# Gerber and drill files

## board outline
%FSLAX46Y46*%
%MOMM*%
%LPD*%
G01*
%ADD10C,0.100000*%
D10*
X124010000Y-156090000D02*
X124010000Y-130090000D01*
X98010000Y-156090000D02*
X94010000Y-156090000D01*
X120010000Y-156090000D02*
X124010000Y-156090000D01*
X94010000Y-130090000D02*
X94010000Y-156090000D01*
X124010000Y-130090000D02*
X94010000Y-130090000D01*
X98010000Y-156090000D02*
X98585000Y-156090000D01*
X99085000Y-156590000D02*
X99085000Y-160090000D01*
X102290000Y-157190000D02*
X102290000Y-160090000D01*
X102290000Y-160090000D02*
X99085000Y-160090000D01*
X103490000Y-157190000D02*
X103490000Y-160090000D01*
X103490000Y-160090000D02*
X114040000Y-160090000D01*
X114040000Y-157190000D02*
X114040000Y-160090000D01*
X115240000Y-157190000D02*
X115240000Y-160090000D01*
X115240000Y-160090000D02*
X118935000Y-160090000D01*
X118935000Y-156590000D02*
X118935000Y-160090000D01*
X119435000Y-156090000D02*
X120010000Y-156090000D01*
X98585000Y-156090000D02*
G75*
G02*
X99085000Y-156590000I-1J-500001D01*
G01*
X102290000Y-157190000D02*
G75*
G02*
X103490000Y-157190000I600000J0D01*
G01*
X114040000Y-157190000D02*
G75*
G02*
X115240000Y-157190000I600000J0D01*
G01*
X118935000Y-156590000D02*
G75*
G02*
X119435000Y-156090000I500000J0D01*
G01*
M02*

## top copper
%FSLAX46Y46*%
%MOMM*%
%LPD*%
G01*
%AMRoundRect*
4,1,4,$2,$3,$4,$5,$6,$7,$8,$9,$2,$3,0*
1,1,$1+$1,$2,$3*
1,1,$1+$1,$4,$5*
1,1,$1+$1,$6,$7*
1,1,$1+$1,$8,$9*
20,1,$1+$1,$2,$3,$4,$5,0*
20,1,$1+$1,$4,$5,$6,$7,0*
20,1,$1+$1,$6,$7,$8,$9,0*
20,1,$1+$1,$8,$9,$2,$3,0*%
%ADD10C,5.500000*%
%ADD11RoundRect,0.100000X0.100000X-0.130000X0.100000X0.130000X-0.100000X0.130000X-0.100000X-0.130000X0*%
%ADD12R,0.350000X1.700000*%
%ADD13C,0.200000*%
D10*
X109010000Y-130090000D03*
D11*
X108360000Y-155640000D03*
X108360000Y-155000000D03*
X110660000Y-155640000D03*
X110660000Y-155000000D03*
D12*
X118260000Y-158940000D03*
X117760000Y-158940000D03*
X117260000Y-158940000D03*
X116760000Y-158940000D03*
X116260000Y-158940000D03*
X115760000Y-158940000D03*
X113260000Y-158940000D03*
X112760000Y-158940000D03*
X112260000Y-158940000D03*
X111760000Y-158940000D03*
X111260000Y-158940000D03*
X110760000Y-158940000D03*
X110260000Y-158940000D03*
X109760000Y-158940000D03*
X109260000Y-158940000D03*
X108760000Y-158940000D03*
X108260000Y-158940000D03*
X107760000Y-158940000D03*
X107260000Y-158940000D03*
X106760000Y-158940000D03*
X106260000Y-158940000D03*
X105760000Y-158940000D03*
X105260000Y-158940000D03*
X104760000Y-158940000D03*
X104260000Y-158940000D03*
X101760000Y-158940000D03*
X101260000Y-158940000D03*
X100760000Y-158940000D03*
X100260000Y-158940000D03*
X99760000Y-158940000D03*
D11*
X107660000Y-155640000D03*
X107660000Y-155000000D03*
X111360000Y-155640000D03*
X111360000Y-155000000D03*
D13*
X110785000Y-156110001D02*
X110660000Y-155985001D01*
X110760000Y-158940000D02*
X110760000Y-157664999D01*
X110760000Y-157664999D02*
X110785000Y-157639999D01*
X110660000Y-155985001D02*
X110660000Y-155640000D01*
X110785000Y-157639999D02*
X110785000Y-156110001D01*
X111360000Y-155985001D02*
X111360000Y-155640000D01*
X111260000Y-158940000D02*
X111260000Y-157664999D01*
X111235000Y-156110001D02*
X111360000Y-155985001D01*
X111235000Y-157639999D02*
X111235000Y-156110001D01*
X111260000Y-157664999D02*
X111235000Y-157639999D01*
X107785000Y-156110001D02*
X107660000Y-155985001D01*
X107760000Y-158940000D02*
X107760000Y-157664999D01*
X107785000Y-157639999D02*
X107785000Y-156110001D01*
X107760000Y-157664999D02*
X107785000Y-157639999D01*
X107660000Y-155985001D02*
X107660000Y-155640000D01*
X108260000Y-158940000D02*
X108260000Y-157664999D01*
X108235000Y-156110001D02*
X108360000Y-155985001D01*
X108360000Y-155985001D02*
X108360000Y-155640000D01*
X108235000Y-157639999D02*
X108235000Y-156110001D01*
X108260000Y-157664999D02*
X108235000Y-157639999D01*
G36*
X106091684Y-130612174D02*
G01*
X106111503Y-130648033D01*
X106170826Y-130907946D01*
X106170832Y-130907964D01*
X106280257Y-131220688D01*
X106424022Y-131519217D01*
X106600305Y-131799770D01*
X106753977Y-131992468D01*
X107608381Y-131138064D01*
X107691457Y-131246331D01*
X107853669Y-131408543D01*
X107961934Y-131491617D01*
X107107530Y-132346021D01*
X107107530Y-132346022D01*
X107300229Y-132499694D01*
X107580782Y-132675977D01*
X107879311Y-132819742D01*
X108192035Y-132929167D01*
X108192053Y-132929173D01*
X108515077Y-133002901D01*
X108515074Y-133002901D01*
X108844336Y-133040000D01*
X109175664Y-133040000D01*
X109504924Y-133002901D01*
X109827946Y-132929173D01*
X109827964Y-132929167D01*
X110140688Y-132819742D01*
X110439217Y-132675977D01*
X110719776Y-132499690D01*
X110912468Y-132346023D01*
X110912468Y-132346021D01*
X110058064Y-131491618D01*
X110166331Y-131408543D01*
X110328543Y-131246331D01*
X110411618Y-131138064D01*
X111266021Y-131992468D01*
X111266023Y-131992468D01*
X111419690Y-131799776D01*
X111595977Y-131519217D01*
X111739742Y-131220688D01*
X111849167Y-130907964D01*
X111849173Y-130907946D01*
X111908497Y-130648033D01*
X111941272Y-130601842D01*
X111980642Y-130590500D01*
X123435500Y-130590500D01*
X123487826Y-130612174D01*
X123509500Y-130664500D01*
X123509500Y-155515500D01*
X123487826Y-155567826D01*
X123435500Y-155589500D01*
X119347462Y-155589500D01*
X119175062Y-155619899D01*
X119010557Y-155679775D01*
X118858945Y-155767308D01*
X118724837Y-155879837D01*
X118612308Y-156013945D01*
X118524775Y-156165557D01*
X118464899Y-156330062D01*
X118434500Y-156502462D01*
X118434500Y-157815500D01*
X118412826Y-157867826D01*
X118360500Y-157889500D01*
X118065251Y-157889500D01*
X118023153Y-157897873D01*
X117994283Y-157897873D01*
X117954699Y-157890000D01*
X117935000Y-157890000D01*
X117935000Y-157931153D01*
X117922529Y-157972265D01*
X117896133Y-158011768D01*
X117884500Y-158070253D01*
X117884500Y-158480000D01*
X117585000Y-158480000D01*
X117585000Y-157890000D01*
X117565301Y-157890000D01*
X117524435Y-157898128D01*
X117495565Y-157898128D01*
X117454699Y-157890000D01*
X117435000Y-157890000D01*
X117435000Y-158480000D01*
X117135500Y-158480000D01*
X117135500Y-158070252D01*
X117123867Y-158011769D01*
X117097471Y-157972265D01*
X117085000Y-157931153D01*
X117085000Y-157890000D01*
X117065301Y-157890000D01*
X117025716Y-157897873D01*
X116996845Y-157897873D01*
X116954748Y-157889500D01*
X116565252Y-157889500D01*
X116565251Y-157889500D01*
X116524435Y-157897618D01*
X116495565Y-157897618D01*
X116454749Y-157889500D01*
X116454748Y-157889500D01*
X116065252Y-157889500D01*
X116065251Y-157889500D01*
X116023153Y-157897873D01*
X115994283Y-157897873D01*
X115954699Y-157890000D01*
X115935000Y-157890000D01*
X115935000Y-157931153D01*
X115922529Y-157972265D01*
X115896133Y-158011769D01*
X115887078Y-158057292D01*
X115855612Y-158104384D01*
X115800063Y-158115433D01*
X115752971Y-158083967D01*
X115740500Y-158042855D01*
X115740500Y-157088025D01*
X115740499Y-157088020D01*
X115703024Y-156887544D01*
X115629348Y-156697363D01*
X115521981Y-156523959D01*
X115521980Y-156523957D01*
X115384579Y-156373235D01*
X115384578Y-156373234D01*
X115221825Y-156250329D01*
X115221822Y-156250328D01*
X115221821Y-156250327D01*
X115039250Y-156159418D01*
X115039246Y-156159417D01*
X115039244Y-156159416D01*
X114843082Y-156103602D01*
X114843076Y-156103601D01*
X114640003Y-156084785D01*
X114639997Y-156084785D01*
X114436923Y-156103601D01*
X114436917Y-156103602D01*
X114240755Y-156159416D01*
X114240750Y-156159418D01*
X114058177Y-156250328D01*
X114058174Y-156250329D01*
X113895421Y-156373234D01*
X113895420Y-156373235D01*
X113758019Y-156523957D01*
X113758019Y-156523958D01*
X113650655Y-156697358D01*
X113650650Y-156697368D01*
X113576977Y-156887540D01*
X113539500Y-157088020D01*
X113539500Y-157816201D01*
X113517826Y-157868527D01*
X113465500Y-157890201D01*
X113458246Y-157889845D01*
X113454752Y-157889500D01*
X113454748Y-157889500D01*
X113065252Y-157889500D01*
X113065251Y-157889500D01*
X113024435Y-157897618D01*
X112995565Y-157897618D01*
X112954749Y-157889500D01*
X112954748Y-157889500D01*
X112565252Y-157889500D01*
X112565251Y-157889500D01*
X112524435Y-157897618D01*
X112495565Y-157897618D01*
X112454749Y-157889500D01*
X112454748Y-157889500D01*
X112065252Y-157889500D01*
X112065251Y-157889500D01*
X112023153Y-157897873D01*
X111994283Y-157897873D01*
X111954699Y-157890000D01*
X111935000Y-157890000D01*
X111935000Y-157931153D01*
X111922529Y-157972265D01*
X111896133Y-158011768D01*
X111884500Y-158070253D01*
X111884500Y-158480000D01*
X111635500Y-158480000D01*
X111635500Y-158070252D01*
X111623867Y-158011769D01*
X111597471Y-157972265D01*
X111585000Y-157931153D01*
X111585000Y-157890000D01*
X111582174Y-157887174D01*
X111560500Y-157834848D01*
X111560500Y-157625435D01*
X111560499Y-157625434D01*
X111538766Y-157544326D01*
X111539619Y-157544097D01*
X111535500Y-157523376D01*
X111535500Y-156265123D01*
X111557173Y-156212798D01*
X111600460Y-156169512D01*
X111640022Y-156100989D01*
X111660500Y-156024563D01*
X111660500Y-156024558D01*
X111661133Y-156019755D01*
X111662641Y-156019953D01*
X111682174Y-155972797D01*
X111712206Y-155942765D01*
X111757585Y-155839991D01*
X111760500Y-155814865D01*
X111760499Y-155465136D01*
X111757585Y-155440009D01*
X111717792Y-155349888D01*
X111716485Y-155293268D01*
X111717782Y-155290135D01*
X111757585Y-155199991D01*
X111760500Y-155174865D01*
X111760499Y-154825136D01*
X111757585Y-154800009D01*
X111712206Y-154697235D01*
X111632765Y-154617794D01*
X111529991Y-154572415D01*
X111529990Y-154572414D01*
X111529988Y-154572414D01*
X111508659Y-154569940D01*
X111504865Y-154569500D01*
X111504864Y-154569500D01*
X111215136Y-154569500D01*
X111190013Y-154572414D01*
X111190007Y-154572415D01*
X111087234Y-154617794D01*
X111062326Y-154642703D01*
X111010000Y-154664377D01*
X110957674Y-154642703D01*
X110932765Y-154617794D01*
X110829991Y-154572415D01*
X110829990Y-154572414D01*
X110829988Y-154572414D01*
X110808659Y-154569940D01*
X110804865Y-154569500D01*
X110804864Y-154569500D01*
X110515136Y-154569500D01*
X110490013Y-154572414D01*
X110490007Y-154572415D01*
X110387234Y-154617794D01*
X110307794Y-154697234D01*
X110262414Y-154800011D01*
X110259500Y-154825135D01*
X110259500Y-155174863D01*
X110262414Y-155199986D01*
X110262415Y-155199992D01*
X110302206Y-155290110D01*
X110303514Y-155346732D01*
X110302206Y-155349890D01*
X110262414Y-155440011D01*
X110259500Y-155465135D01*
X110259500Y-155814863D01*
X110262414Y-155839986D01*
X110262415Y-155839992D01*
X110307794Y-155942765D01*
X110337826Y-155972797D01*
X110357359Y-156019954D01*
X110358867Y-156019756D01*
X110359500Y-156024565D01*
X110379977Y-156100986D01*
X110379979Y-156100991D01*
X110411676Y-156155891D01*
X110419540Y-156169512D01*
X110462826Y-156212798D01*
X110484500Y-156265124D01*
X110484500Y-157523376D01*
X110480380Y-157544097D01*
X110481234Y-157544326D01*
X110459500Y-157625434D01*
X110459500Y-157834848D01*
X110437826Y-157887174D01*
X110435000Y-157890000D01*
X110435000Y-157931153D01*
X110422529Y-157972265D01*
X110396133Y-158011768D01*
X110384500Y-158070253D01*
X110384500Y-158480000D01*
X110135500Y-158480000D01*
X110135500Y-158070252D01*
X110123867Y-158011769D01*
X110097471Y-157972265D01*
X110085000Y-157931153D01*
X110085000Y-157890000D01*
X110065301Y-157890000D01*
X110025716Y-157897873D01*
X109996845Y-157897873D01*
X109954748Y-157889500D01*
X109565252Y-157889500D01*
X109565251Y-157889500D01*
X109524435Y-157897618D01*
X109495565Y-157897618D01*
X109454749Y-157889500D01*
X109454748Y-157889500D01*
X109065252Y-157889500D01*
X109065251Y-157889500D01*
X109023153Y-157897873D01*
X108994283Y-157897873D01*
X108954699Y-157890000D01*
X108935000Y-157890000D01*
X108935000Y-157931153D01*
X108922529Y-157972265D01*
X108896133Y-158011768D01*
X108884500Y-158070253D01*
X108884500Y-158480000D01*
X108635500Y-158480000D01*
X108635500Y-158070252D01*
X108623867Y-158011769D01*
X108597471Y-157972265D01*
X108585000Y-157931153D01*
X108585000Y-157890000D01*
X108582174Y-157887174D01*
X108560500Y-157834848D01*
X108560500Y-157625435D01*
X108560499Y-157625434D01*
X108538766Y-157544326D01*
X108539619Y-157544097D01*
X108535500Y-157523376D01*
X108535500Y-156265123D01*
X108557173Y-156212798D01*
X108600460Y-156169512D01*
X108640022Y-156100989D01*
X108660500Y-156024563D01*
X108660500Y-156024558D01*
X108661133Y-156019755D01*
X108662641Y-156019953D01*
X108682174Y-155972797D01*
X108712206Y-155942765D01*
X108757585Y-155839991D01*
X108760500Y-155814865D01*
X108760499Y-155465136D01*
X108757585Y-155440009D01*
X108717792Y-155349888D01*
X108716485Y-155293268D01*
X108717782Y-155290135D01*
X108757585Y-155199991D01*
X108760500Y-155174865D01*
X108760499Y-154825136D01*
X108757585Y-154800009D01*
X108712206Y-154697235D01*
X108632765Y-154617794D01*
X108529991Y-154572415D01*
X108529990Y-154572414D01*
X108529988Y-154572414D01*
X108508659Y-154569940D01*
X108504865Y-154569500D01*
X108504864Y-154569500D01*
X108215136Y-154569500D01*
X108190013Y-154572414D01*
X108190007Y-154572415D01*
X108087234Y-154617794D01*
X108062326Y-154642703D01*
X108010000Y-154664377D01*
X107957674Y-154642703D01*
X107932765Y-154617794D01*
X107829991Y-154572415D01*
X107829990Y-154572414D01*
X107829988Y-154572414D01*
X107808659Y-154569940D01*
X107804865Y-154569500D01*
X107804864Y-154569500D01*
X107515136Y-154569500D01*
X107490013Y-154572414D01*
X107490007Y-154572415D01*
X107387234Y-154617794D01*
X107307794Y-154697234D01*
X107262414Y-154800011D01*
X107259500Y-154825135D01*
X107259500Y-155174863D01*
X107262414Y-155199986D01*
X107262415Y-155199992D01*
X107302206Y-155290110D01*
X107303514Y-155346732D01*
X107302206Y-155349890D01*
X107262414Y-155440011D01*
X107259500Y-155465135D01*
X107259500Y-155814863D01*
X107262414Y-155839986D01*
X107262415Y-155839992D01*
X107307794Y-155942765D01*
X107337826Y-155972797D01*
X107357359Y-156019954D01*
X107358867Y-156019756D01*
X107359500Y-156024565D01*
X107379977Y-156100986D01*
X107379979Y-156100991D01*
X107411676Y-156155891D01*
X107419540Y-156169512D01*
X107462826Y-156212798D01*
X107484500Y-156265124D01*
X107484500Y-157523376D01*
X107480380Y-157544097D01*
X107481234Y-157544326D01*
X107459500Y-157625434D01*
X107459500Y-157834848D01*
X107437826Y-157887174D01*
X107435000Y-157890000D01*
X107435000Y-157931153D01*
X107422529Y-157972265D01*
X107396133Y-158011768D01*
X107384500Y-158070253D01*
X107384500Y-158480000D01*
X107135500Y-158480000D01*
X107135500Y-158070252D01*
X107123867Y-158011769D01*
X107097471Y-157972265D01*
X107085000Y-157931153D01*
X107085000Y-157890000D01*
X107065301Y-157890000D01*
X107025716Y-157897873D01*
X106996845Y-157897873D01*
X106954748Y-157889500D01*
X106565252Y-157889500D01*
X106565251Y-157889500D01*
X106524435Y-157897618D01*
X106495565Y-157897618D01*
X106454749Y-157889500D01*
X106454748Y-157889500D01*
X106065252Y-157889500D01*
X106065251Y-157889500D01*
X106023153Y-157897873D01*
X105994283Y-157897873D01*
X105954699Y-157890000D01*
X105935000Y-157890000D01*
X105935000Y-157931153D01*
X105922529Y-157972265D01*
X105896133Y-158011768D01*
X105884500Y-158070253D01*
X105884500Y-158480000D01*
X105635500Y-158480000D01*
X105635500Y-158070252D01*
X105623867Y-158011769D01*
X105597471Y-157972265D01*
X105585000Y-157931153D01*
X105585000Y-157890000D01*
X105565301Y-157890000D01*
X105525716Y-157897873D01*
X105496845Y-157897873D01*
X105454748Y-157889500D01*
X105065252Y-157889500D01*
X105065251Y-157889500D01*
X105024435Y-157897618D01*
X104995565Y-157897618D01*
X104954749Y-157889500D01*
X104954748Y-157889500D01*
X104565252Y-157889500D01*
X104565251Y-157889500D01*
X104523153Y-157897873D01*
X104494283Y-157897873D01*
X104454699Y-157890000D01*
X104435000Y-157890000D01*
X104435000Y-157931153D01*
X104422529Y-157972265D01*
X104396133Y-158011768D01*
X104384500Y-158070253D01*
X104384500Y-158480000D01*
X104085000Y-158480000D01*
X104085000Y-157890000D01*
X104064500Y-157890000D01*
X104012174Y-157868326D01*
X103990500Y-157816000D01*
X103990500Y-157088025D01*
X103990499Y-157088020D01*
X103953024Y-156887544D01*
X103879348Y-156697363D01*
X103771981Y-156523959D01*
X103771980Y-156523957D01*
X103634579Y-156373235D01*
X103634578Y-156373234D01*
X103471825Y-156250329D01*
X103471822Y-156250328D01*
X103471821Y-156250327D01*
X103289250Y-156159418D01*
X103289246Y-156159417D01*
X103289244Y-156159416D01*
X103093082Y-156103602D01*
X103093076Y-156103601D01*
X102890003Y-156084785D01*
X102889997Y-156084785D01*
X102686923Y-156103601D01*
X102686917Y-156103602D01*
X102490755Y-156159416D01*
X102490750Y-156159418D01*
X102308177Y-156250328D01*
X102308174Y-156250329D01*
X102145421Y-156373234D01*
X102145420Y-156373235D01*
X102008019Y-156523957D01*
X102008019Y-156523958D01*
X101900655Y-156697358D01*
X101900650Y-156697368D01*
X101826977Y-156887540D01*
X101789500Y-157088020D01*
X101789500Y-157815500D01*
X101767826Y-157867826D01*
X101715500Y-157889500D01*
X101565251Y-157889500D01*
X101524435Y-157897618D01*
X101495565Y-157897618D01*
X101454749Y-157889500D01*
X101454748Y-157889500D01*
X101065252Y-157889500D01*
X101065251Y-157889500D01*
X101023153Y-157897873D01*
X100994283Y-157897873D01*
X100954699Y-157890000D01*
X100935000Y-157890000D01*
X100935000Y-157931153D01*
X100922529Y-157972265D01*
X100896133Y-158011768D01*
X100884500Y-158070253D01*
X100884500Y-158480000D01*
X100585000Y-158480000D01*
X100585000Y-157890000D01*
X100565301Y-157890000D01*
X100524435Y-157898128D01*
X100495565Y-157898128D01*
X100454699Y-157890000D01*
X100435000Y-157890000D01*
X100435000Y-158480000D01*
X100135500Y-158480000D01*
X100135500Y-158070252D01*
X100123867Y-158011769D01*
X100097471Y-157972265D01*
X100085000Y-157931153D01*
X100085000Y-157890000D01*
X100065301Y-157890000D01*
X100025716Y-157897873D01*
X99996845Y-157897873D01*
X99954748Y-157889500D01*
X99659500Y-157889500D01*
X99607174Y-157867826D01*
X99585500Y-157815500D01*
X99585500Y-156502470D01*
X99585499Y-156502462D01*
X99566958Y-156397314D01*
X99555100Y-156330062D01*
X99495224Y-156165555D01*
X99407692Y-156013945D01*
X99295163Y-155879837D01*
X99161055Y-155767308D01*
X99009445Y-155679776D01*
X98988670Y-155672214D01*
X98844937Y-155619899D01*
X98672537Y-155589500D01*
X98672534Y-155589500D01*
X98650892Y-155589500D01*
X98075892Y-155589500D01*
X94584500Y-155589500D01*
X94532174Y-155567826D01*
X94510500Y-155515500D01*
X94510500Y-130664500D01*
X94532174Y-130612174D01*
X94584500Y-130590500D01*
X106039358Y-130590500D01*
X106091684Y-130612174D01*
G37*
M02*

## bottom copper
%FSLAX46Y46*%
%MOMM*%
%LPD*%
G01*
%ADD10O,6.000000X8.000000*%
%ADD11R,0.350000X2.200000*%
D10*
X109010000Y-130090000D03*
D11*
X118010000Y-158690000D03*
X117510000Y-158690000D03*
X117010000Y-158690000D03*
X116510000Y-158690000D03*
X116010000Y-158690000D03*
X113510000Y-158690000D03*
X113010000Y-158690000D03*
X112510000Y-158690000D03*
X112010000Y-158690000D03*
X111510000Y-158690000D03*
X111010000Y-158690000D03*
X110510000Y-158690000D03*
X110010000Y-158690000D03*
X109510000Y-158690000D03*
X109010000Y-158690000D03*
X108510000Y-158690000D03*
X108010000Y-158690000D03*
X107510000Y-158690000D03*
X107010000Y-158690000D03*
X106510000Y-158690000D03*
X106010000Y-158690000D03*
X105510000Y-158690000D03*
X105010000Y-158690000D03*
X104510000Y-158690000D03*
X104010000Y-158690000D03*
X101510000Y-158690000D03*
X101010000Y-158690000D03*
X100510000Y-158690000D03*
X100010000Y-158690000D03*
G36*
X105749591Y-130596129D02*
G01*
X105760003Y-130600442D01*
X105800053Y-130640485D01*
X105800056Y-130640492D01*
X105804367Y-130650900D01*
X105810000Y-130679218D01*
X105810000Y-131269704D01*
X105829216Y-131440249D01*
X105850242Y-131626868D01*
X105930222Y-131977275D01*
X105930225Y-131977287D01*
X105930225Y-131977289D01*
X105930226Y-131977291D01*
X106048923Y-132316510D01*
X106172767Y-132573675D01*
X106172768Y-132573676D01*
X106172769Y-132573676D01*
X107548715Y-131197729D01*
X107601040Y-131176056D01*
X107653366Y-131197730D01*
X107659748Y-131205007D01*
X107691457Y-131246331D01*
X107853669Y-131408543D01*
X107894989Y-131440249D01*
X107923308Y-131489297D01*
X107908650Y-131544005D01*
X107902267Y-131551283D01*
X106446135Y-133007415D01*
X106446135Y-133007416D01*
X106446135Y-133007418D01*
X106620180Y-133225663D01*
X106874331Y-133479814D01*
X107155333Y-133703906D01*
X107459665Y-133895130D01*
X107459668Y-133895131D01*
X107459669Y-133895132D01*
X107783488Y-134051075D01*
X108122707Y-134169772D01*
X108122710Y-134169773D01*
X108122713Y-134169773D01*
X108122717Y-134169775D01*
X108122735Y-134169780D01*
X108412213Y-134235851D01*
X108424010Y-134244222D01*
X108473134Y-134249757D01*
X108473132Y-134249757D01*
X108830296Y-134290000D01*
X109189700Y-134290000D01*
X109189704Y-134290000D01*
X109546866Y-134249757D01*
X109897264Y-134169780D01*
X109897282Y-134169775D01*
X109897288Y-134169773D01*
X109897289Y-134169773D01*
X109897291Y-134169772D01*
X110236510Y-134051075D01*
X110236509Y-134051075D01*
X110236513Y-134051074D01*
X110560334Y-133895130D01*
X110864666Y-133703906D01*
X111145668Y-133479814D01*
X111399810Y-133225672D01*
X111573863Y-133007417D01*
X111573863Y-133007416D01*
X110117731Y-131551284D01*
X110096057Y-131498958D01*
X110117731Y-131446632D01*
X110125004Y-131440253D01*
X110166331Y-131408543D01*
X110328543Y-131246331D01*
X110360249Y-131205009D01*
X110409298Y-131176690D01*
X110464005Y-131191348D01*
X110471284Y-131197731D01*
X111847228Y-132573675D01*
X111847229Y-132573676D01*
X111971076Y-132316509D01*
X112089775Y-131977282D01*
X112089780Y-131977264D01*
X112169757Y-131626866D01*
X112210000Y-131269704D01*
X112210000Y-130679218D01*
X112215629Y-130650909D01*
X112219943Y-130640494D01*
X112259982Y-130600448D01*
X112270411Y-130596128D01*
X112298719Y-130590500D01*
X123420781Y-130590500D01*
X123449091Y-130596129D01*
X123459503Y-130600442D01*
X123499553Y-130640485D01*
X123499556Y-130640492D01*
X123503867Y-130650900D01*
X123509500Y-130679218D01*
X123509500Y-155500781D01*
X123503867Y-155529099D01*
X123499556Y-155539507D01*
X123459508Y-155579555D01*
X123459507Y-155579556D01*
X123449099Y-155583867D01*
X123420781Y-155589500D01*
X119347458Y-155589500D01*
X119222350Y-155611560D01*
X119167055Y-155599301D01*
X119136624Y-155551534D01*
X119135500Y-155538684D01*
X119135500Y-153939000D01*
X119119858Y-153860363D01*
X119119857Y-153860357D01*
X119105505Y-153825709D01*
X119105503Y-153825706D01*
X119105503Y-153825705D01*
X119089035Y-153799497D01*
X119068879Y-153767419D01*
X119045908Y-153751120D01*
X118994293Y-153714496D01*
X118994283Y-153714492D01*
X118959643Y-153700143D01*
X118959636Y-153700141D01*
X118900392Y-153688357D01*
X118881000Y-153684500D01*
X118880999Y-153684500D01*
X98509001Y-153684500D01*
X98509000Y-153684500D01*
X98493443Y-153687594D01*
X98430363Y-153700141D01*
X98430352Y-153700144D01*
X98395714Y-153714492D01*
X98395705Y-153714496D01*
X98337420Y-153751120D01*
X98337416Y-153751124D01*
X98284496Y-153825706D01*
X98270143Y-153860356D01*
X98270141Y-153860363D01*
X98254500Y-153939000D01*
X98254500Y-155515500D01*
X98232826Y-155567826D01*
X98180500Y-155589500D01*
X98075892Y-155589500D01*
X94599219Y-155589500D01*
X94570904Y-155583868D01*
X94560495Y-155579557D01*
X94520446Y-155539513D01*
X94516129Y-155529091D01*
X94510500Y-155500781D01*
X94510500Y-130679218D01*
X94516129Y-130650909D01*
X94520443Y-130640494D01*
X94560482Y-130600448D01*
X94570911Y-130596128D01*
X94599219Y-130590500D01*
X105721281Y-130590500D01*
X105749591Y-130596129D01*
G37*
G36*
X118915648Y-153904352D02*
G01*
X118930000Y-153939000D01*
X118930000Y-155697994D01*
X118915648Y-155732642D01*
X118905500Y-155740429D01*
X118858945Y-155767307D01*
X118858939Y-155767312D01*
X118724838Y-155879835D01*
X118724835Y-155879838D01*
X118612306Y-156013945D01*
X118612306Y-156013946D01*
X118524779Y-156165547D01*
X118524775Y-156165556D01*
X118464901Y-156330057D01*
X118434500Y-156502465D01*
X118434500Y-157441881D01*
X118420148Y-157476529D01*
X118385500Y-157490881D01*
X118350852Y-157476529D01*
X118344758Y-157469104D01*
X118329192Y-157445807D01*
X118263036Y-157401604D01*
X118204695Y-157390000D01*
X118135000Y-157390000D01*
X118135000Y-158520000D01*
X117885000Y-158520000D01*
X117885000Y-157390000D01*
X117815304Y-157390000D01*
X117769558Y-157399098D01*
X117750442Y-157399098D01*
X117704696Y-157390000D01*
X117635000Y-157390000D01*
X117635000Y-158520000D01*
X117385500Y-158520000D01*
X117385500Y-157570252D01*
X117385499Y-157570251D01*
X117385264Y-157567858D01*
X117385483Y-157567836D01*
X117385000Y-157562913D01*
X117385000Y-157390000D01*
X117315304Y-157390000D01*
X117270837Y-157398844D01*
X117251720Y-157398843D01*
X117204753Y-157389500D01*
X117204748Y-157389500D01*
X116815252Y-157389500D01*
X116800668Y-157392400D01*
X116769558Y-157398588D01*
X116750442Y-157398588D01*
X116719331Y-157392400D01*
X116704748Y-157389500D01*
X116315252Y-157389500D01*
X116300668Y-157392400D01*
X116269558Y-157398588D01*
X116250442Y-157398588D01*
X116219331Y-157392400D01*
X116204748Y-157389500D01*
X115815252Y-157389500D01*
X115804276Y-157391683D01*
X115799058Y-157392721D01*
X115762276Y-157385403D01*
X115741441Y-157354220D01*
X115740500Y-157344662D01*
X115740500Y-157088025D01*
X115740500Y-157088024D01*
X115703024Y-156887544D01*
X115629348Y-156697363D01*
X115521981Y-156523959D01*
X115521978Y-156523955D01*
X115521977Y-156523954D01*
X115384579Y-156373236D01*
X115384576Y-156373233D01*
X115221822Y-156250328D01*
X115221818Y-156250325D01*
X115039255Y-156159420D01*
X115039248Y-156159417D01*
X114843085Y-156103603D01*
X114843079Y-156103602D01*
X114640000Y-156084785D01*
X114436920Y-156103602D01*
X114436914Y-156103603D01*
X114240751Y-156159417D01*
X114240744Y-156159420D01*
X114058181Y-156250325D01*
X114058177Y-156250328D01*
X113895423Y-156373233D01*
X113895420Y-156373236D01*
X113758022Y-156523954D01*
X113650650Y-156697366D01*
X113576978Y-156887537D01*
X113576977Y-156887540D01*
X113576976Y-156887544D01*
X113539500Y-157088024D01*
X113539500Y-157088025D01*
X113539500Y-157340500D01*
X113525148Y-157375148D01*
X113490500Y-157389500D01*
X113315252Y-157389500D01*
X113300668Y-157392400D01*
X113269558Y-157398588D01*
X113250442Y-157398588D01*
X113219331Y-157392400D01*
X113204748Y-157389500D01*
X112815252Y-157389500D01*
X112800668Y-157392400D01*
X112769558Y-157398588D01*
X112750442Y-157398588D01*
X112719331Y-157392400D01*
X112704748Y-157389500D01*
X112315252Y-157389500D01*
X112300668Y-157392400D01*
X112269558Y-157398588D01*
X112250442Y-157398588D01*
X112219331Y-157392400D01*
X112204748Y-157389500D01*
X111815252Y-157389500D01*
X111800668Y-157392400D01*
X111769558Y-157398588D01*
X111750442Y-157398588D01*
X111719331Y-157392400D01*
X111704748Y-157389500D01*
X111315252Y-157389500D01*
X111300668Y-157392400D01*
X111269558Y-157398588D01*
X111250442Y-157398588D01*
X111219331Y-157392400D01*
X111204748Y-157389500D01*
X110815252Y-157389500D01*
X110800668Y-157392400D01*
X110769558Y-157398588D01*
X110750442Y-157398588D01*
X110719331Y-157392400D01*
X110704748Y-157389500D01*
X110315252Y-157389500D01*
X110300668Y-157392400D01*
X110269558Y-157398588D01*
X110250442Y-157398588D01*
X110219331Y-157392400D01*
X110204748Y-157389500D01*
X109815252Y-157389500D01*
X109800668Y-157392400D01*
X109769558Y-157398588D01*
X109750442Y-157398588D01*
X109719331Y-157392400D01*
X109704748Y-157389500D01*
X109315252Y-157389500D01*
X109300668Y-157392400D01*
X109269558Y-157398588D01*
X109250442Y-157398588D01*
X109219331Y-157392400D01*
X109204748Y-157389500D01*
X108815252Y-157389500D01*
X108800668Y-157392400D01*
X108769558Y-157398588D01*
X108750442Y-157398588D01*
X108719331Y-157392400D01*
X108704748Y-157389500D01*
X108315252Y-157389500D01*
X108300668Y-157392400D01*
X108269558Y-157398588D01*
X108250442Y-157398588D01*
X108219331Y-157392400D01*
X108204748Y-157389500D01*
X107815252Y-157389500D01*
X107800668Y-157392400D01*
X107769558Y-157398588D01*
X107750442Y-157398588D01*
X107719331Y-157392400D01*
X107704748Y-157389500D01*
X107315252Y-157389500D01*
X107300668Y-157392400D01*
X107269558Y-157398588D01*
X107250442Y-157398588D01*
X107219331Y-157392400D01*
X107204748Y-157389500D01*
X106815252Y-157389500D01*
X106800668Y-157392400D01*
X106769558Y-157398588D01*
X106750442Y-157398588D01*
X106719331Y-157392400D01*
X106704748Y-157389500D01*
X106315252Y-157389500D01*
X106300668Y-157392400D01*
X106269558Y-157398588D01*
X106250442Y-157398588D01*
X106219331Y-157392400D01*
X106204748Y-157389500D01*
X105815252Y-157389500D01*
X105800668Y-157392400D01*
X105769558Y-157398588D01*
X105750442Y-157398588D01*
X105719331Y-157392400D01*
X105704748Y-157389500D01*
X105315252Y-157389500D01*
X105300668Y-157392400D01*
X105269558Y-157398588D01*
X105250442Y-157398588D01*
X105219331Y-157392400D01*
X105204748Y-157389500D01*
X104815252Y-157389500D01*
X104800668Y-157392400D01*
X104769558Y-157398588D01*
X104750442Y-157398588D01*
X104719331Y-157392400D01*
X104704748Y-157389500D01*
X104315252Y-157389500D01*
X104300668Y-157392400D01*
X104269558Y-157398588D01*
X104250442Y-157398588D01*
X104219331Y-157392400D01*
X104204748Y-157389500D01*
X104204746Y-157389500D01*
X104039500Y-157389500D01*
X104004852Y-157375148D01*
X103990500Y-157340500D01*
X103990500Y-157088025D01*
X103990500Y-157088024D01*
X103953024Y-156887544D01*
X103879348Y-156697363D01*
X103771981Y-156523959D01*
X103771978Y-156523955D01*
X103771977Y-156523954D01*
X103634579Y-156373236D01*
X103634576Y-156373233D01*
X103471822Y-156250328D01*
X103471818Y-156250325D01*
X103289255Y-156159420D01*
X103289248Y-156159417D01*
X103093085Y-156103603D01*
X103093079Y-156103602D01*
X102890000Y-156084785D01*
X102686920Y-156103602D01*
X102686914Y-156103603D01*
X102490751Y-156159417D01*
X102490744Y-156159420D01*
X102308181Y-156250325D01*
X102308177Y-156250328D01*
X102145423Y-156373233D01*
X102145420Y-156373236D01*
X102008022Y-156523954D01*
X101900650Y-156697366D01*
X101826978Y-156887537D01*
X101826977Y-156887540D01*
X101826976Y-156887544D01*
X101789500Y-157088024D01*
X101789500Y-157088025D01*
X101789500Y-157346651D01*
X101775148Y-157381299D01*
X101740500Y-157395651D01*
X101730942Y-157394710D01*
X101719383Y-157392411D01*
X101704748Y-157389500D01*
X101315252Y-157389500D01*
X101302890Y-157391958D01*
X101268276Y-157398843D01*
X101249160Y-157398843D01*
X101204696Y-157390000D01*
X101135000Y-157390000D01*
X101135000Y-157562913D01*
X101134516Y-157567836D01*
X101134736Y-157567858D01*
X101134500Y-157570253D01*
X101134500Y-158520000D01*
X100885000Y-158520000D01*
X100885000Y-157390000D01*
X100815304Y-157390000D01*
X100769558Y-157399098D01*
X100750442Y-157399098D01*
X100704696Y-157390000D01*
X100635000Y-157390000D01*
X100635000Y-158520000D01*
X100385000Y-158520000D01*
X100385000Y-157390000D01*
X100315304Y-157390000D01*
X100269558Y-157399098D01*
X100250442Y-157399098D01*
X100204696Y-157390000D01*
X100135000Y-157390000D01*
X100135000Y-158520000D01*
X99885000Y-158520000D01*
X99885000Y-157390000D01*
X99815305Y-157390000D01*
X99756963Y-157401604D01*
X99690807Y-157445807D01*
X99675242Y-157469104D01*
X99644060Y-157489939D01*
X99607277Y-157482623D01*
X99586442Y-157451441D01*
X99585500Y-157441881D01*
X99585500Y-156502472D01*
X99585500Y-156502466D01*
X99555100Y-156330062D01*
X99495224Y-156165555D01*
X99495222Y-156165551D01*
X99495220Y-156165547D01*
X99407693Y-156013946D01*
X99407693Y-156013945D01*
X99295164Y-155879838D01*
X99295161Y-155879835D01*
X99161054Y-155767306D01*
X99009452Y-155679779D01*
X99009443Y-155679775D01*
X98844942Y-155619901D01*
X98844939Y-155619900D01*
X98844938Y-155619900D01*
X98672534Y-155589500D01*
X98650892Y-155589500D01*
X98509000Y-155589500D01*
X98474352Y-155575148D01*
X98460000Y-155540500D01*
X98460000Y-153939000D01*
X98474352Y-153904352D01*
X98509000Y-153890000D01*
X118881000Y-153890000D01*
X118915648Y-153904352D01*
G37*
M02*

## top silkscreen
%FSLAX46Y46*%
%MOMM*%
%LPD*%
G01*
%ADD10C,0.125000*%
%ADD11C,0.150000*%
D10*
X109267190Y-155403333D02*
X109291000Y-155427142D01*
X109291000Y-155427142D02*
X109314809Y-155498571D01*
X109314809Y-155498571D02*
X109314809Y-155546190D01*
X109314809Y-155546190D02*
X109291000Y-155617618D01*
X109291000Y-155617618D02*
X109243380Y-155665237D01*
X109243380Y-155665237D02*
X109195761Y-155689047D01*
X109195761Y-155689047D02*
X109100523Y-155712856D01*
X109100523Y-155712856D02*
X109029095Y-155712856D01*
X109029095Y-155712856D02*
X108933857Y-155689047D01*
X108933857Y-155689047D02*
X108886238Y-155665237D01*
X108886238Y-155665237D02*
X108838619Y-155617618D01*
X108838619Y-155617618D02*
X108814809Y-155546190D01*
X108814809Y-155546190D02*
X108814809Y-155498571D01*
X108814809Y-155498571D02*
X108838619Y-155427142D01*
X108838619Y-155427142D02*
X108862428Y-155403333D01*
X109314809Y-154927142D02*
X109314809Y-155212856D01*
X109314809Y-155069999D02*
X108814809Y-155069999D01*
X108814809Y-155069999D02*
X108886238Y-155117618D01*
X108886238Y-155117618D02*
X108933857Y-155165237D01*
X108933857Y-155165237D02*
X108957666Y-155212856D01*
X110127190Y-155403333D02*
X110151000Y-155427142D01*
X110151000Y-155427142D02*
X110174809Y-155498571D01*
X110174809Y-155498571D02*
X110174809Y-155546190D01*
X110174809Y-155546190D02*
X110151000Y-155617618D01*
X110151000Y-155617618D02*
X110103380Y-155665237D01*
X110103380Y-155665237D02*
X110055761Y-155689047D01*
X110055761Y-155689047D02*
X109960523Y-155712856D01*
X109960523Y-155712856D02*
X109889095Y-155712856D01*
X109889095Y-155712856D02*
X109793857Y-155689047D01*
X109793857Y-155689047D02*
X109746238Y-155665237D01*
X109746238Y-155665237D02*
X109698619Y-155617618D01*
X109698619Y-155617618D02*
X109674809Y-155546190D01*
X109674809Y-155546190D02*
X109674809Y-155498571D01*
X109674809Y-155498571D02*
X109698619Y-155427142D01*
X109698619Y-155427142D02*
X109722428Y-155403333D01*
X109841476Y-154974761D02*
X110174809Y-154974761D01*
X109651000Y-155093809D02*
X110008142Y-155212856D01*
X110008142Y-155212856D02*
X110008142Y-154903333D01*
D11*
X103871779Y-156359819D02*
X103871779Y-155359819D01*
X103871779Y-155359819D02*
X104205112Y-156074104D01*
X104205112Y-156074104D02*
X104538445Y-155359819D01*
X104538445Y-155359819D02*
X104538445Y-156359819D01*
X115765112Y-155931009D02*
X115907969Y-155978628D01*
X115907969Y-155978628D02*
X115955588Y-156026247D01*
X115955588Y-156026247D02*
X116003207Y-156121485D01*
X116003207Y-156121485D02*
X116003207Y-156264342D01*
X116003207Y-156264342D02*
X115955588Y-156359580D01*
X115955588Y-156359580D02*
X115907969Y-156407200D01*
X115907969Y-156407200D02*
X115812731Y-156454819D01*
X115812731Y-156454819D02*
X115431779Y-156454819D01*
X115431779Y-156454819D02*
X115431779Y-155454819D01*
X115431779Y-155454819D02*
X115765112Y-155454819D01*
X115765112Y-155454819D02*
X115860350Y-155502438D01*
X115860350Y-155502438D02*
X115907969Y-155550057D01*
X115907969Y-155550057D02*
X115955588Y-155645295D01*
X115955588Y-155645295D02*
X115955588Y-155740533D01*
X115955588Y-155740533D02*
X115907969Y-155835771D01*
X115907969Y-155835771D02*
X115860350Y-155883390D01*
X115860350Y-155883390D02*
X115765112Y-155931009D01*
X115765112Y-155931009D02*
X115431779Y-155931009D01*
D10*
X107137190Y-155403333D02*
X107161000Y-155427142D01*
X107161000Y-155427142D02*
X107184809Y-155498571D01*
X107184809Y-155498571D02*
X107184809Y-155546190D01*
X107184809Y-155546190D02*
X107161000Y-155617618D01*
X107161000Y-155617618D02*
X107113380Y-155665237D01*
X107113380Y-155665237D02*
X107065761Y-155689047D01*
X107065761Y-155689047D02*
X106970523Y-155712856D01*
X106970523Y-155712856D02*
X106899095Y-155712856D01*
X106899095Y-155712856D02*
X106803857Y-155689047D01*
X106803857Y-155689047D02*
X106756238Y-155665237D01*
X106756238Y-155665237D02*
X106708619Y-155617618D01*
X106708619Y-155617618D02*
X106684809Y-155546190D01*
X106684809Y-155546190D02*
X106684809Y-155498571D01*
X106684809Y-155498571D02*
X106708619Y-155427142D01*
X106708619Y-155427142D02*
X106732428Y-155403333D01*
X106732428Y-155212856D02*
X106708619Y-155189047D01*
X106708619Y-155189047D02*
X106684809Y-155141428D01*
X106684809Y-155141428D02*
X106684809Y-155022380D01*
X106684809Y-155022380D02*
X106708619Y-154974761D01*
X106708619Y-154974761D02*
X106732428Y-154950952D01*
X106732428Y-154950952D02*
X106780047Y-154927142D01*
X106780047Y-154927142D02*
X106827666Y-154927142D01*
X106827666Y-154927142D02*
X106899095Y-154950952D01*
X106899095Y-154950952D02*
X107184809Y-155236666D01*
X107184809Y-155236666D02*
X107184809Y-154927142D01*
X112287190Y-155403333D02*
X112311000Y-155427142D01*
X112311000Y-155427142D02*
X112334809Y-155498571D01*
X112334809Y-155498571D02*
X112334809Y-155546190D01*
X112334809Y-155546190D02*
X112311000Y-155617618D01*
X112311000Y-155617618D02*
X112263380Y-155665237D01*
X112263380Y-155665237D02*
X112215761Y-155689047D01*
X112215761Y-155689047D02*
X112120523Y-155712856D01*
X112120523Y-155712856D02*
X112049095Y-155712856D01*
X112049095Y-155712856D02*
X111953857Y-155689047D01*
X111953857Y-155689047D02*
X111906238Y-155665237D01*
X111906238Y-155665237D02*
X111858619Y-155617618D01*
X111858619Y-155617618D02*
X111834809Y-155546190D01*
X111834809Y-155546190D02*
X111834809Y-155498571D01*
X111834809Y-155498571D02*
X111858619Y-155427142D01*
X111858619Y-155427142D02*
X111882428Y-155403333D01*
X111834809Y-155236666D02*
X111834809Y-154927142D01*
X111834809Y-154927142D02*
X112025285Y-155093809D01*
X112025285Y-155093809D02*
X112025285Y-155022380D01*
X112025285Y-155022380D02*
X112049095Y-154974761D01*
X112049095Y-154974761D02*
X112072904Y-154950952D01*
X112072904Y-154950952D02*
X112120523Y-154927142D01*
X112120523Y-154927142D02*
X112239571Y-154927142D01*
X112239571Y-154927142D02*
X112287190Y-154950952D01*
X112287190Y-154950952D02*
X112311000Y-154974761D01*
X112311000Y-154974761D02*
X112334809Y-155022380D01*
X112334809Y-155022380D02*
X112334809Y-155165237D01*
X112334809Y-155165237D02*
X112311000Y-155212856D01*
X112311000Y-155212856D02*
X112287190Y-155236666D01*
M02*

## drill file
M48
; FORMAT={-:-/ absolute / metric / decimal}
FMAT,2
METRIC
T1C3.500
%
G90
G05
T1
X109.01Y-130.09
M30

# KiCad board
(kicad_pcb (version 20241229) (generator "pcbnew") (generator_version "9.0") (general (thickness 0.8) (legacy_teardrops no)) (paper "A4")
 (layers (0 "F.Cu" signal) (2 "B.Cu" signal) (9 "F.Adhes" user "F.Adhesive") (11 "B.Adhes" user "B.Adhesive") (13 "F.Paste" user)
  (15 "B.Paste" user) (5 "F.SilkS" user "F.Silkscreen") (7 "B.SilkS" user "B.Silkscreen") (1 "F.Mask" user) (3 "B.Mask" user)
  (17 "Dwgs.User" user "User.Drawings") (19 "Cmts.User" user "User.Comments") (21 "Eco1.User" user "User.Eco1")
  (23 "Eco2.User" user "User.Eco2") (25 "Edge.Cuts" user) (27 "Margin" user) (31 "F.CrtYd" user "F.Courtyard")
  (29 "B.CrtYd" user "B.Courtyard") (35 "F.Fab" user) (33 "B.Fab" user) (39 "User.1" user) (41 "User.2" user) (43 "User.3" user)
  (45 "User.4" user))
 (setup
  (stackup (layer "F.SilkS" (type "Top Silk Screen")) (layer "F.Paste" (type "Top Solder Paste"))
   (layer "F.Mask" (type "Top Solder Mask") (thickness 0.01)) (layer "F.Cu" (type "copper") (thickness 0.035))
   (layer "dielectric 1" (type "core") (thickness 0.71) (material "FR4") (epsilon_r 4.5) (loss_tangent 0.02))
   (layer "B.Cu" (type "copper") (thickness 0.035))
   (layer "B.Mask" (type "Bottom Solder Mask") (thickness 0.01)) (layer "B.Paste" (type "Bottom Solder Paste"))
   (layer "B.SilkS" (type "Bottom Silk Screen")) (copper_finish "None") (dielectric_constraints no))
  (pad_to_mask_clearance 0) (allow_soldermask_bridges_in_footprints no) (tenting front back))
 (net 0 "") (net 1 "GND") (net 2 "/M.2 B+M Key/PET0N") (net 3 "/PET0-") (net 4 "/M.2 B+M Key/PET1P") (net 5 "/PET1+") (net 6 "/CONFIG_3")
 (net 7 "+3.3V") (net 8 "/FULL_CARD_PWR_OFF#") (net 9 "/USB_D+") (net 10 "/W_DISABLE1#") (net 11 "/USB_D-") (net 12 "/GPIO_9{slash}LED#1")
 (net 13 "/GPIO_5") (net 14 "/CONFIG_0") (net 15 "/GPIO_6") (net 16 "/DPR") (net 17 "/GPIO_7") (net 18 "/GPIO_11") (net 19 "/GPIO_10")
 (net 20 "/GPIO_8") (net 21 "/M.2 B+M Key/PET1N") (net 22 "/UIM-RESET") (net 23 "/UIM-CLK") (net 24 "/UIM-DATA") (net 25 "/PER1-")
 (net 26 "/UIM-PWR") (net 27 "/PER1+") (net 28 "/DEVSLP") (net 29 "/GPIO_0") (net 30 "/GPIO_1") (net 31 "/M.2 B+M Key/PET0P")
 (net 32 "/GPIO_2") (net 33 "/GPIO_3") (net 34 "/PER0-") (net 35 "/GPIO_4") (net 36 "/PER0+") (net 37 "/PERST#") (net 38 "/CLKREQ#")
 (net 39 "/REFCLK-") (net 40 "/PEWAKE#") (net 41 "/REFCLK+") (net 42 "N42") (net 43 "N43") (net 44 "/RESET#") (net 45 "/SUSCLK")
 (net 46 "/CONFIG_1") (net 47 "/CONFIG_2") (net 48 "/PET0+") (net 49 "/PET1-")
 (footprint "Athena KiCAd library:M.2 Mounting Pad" (layer "F.Cu") (at 109.01 130.09)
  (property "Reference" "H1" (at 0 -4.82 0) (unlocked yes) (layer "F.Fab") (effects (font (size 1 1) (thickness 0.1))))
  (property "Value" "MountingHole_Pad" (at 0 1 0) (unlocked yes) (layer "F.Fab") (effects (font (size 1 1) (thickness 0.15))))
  (pad "1" thru_hole circle (at 0 0) (size 5.5 5.5) (drill 3.5) (layers "*.Cu" "*.Mask") (remove_unused_layers no) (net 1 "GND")
   (padstack (mode front_inner_back)
    (layer "Inner" (shape circle) (size 5.5 5.5) (zone_connect -1))
    (layer "B.Cu" (shape oval) (size 6 8) (thermal_bridge_angle 45) (zone_connect -1)))))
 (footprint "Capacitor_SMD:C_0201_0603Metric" (layer "F.Cu") (at 108.36 155.32 90)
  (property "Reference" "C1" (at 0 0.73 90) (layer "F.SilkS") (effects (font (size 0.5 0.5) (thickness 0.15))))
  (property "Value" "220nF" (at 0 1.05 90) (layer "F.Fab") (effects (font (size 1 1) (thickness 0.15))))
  (pad "" smd roundrect (at -0.345 0 90) (size 0.318 0.36) (layers "F.Paste") (roundrect_rratio 0.25))
  (pad "" smd roundrect (at 0.345 0 90) (size 0.318 0.36) (layers "F.Paste") (roundrect_rratio 0.25))
  (pad "1" smd roundrect (at -0.32 0 90) (size 0.46 0.4) (layers "F.Cu" "F.Mask") (roundrect_rratio 0.25) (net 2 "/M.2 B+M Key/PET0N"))
  (pad "2" smd roundrect (at 0.32 0 90) (size 0.46 0.4) (layers "F.Cu" "F.Mask") (roundrect_rratio 0.25) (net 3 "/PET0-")))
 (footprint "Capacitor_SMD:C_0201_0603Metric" (layer "F.Cu") (at 110.66 155.32 90)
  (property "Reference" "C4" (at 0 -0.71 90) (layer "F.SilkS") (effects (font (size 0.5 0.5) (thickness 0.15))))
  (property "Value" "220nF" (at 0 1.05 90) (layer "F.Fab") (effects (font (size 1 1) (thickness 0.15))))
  (pad "" smd roundrect (at -0.345 0 90) (size 0.318 0.36) (layers "F.Paste") (roundrect_rratio 0.25))
  (pad "" smd roundrect (at 0.345 0 90) (size 0.318 0.36) (layers "F.Paste") (roundrect_rratio 0.25))
  (pad "1" smd roundrect (at -0.32 0 90) (size 0.46 0.4) (layers "F.Cu" "F.Mask") (roundrect_rratio 0.25) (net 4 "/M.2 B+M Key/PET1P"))
  (pad "2" smd roundrect (at 0.32 0 90) (size 0.46 0.4) (layers "F.Cu" "F.Mask") (roundrect_rratio 0.25) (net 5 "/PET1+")))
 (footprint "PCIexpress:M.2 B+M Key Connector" (layer "F.Cu") (at 109.01 158.98)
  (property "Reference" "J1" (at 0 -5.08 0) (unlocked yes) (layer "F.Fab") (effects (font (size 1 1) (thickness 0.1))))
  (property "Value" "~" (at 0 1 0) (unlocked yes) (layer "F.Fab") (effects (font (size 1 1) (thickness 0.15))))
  (fp_line (start -11 -2.89) (end -10.425 -2.89) (stroke (width 0.1) (type default)) (layer "Edge.Cuts") (net 4))
  (fp_line (start -9.925 -2.39) (end -9.925 1.11) (stroke (width 0.1) (type default)) (layer "Edge.Cuts") (net 4))
  (fp_line (start -6.72 -1.79) (end -6.72 1.11) (stroke (width 0.1) (type default)) (layer "Edge.Cuts") (net 4))
  (fp_line (start -6.72 1.11) (end -9.925 1.11) (stroke (width 0.1) (type default)) (layer "Edge.Cuts") (net 4))
  (fp_line (start -5.52 -1.79) (end -5.52 1.11) (stroke (width 0.1) (type default)) (layer "Edge.Cuts") (net 4))
  (fp_line (start -5.52 1.11) (end 5.03 1.11) (stroke (width 0.1) (type default)) (layer "Edge.Cuts") (net 4))
  (fp_line (start 5.03 -1.79) (end 5.03 1.11) (stroke (width 0.1) (type default)) (layer "Edge.Cuts") (net 4))
  (fp_line (start 6.23 -1.79) (end 6.23 1.11) (stroke (width 0.1) (type default)) (layer "Edge.Cuts") (net 4))
  (fp_line (start 6.23 1.11) (end 9.925 1.11) (stroke (width 0.1) (type default)) (layer "Edge.Cuts") (net 4))
  (fp_line (start 9.925 -2.39) (end 9.925 1.11) (stroke (width 0.1) (type default)) (layer "Edge.Cuts") (net 4))
  (fp_line (start 10.425 -2.89) (end 11 -2.89) (stroke (width 0.1) (type default)) (layer "Edge.Cuts") (net 4))
  (fp_arc (start -10.425 -2.89) (mid -10.071447 -2.743553) (end -9.925 -2.39) (stroke (width 0.1) (type default)) (layer "Edge.Cuts")
   (net 4))
  (fp_arc (start -6.72 -1.79) (mid -6.12 -2.39) (end -5.52 -1.79) (stroke (width 0.1) (type default)) (layer "Edge.Cuts") (net 4))
  (fp_arc (start 5.03 -1.79) (mid 5.63 -2.39) (end 6.23 -1.79) (stroke (width 0.1) (type default)) (layer "Edge.Cuts") (net 4))
  (fp_arc (start 9.925 -2.39) (mid 10.071447 -2.743553) (end 10.425 -2.89) (stroke (width 0.1) (type default)) (layer "Edge.Cuts") (net 4))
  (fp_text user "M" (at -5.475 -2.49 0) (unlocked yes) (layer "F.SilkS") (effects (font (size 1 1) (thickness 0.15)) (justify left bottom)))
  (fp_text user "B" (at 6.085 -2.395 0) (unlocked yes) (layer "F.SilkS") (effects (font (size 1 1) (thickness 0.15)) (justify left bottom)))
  (pad "1" smd rect (at 9.25 -0.04 180) (size 0.35 1.7) (layers "F.Cu") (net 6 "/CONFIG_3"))
  (pad "2" smd rect (at 9 -0.29 180) (size 0.35 2.2) (layers "B.Cu") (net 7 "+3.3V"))
  (pad "3" smd rect (at 8.75 -0.04 180) (size 0.35 1.7) (layers "F.Cu") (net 1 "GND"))
  (pad "4" smd rect (at 8.5 -0.29 180) (size 0.35 2.2) (layers "B.Cu") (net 7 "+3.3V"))
  (pad "5" smd rect (at 8.25 -0.04 180) (size 0.35 1.7) (layers "F.Cu") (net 1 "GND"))
  (pad "6" smd rect (at 8 -0.29 180) (size 0.35 2.2) (layers "B.Cu") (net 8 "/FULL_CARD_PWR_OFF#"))
  (pad "7" smd rect (at 7.75 -0.04 180) (size 0.35 1.7) (layers "F.Cu") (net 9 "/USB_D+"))
  (pad "8" smd rect (at 7.5 -0.29 180) (size 0.35 2.2) (layers "B.Cu") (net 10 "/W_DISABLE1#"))
  (pad "9" smd rect (at 7.25 -0.04 180) (size 0.35 1.7) (layers "F.Cu") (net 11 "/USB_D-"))
  (pad "10" smd rect (at 7 -0.29 180) (size 0.35 2.2) (layers "B.Cu") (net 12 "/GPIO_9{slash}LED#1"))
  (pad "11" smd rect (at 6.75 -0.04 180) (size 0.35 1.7) (layers "F.Cu") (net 1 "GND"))
  (pad "20" smd rect (at 4.5 -0.29 180) (size 0.35 2.2) (layers "B.Cu") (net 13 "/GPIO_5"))
  (pad "21" smd rect (at 4.25 -0.04 180) (size 0.35 1.7) (layers "F.Cu") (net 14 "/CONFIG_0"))
  (pad "22" smd rect (at 4 -0.29 180) (size 0.35 2.2) (layers "B.Cu") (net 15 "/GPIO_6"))
  (pad "23" smd rect (at 3.75 -0.04 180) (size 0.35 1.7) (layers "F.Cu") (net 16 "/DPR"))
  (pad "24" smd rect (at 3.5 -0.29 180) (size 0.35 2.2) (layers "B.Cu") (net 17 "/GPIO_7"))
  (pad "25" smd rect (at 3.25 -0.04 180) (size 0.35 1.7) (layers "F.Cu") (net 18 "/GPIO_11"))
  (pad "26" smd rect (at 3 -0.29 180) (size 0.35 2.2) (layers "B.Cu") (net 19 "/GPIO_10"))
  (pad "27" smd rect (at 2.75 -0.04 180) (size 0.35 1.7) (layers "F.Cu") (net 1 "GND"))
  (pad "28" smd rect (at 2.5 -0.29 180) (size 0.35 2.2) (layers "B.Cu") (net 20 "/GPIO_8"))
  (pad "29" smd rect (at 2.25 -0.04 180) (size 0.35 1.7) (layers "F.Cu") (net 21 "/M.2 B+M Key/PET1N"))
  (pad "30" smd rect (at 2 -0.29 180) (size 0.35 2.2) (layers "B.Cu") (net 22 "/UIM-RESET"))
  (pad "31" smd rect (at 1.75 -0.04 180) (size 0.35 1.7) (layers "F.Cu") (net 4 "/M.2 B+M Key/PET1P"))
  (pad "32" smd rect (at 1.5 -0.29 180) (size 0.35 2.2) (layers "B.Cu") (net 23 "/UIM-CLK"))
  (pad "33" smd rect (at 1.25 -0.04 180) (size 0.35 1.7) (layers "F.Cu") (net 1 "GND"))
  (pad "34" smd rect (at 1 -0.29 180) (size 0.35 2.2) (layers "B.Cu") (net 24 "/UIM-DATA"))
  (pad "35" smd rect (at 0.75 -0.04 180) (size 0.35 1.7) (layers "F.Cu") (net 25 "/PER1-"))
  (pad "36" smd rect (at 0.5 -0.29 180) (size 0.35 2.2) (layers "B.Cu") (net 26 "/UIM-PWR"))
  (pad "37" smd rect (at 0.25 -0.04 180) (size 0.35 1.7) (layers "F.Cu") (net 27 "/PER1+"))
  (pad "38" smd rect (at 0 -0.29 180) (size 0.35 2.2) (layers "B.Cu") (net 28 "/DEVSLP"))
  (pad "39" smd rect (at -0.25 -0.04 180) (size 0.35 1.7) (layers "F.Cu") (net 1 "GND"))
  (pad "40" smd rect (at -0.5 -0.29 180) (size 0.35 2.2) (layers "B.Cu") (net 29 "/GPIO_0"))
  (pad "41" smd rect (at -0.75 -0.04 180) (size 0.35 1.7) (layers "F.Cu") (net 2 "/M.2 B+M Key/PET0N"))
  (pad "42" smd rect (at -1 -0.29 180) (size 0.35 2.2) (layers "B.Cu") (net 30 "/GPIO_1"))
  (pad "43" smd rect (at -1.25 -0.04 180) (size 0.35 1.7) (layers "F.Cu") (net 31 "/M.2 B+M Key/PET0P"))
  (pad "44" smd rect (at -1.5 -0.29 180) (size 0.35 2.2) (layers "B.Cu") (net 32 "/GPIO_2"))
  (pad "45" smd rect (at -1.75 -0.04 180) (size 0.35 1.7) (layers "F.Cu") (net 1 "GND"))
  (pad "46" smd rect (at -2 -0.29 180) (size 0.35 2.2) (layers "B.Cu") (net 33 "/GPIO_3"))
  (pad "47" smd rect (at -2.25 -0.04 180) (size 0.35 1.7) (layers "F.Cu") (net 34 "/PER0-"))
  (pad "48" smd rect (at -2.5 -0.29 180) (size 0.35 2.2) (layers "B.Cu") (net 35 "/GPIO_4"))
  (pad "49" smd rect (at -2.75 -0.04 180) (size 0.35 1.7) (layers "F.Cu") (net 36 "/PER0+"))
  (pad "50" smd rect (at -3 -0.29 180) (size 0.35 2.2) (layers "B.Cu") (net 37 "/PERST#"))
  (pad "51" smd rect (at -3.25 -0.04 180) (size 0.35 1.7) (layers "F.Cu") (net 1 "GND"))
  (pad "52" smd rect (at -3.5 -0.29 180) (size 0.35 2.2) (layers "B.Cu") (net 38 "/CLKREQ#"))
  (pad "53" smd rect (at -3.75 -0.04 180) (size 0.35 1.7) (layers "F.Cu") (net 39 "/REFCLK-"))
  (pad "54" smd rect (at -4 -0.29 180) (size 0.35 2.2) (layers "B.Cu") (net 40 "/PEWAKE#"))
  (pad "55" smd rect (at -4.25 -0.04 180) (size 0.35 1.7) (layers "F.Cu") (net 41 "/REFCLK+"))
  (pad "56" smd rect (at -4.5 -0.29 180) (size 0.35 2.2) (layers "B.Cu") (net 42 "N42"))
  (pad "57" smd rect (at -4.75 -0.04 180) (size 0.35 1.7) (layers "F.Cu") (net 1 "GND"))
  (pad "58" smd rect (at -5 -0.29 180) (size 0.35 2.2) (layers "B.Cu") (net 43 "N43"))
  (pad "67" smd rect (at -7.25 -0.04 180) (size 0.35 1.7) (layers "F.Cu") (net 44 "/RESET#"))
  (pad "68" smd rect (at -7.5 -0.29 180) (size 0.35 2.2) (layers "B.Cu") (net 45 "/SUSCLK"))
  (pad "69" smd rect (at -7.75 -0.04 180) (size 0.35 1.7) (layers "F.Cu") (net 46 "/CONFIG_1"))
  (pad "70" smd rect (at -8 -0.29 180) (size 0.35 2.2) (layers "B.Cu") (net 7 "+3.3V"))
  (pad "71" smd rect (at -8.25 -0.04 180) (size 0.35 1.7) (layers "F.Cu") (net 1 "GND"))
  (pad "72" smd rect (at -8.5 -0.29 180) (size 0.35 2.2) (layers "B.Cu") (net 7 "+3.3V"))
  (pad "73" smd rect (at -8.75 -0.04 180) (size 0.35 1.7) (layers "F.Cu") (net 1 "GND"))
  (pad "74" smd rect (at -9 -0.29 180) (size 0.35 2.2) (layers "B.Cu") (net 7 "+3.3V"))
  (pad "75" smd rect (at -9.25 -0.04 180) (size 0.35 1.7) (layers "F.Cu") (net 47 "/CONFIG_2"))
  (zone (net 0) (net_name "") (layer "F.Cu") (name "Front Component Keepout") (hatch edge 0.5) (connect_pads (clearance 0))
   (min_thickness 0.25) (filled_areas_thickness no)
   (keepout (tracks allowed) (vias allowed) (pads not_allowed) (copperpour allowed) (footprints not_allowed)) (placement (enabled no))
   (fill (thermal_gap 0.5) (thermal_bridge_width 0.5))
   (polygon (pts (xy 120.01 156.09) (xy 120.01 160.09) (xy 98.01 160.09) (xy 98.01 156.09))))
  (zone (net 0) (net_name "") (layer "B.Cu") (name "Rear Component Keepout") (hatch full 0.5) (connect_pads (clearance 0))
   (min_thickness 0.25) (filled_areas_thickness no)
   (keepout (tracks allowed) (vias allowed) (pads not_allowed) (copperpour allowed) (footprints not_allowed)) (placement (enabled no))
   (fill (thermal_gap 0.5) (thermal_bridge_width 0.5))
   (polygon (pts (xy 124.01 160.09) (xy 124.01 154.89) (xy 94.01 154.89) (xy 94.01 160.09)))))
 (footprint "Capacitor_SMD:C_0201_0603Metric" (layer "F.Cu") (at 107.66 155.32 90)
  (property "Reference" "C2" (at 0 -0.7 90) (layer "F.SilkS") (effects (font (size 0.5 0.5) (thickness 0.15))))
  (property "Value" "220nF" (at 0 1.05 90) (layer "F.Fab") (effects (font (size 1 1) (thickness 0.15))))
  (pad "" smd roundrect (at -0.345 0 90) (size 0.318 0.36) (layers "F.Paste") (roundrect_rratio 0.25))
  (pad "" smd roundrect (at 0.345 0 90) (size 0.318 0.36) (layers "F.Paste") (roundrect_rratio 0.25))
  (pad "1" smd roundrect (at -0.32 0 90) (size 0.46 0.4) (layers "F.Cu" "F.Mask") (roundrect_rratio 0.25) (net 31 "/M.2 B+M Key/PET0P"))
  (pad "2" smd roundrect (at 0.32 0 90) (size 0.46 0.4) (layers "F.Cu" "F.Mask") (roundrect_rratio 0.25) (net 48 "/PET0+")))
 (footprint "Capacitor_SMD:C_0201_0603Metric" (layer "F.Cu") (at 111.36 155.32 90)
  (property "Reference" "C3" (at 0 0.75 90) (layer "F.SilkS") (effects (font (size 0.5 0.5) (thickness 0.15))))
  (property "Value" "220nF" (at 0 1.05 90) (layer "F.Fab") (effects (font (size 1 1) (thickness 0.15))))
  (pad "" smd roundrect (at -0.345 0 90) (size 0.318 0.36) (layers "F.Paste") (roundrect_rratio 0.25))
  (pad "" smd roundrect (at 0.345 0 90) (size 0.318 0.36) (layers "F.Paste") (roundrect_rratio 0.25))
  (pad "1" smd roundrect (at -0.32 0 90) (size 0.46 0.4) (layers "F.Cu" "F.Mask") (roundrect_rratio 0.25) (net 21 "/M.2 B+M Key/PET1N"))
  (pad "2" smd roundrect (at 0.32 0 90) (size 0.46 0.4) (layers "F.Cu" "F.Mask") (roundrect_rratio 0.25) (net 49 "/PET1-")))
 (gr_line (start 124.01 156.09) (end 124.01 130.09) (stroke (width 0.1) (type default)) (layer "Edge.Cuts"))
 (gr_line (start 98.01 156.09) (end 94.01 156.09) (stroke (width 0.1) (type default)) (layer "Edge.Cuts"))
 (gr_line (start 120.01 156.09) (end 124.01 156.09) (stroke (width 0.1) (type default)) (layer "Edge.Cuts"))
 (gr_line (start 94.01 130.09) (end 94.01 156.09) (stroke (width 0.1) (type default)) (layer "Edge.Cuts"))
 (gr_line (start 124.01 130.09) (end 94.01 130.09) (stroke (width 0.1) (type default)) (layer "Edge.Cuts"))
 (segment (start 110.785 156.110001) (end 110.66 155.985001) (width 0.2) (layer "F.Cu") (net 4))
 (segment (start 110.76 158.94) (end 110.76 157.664999) (width 0.2) (layer "F.Cu") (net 4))
 (segment (start 110.76 157.664999) (end 110.785 157.639999) (width 0.2) (layer "F.Cu") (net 4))
 (segment (start 110.66 155.985001) (end 110.66 155.64) (width 0.2) (layer "F.Cu") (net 4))
 (segment (start 110.785 157.639999) (end 110.785 156.110001) (width 0.2) (layer "F.Cu") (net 4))
 (segment (start 111.36 155.985001) (end 111.36 155.64) (width 0.2) (layer "F.Cu") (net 21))
 (segment (start 111.26 158.94) (end 111.26 157.664999) (width 0.2) (layer "F.Cu") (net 21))
 (segment (start 111.235 156.110001) (end 111.36 155.985001) (width 0.2) (layer "F.Cu") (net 21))
 (segment (start 111.235 157.639999) (end 111.235 156.110001) (width 0.2) (layer "F.Cu") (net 21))
 (segment (start 111.26 157.664999) (end 111.235 157.639999) (width 0.2) (layer "F.Cu") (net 21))
 (segment (start 107.785 156.110001) (end 107.66 155.985001) (width 0.2) (layer "F.Cu") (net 31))
 (segment (start 107.76 158.94) (end 107.76 157.664999) (width 0.2) (layer "F.Cu") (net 31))
 (segment (start 107.785 157.639999) (end 107.785 156.110001) (width 0.2) (layer "F.Cu") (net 31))
 (segment (start 107.76 157.664999) (end 107.785 157.639999) (width 0.2) (layer "F.Cu") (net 31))
 (segment (start 107.66 155.985001) (end 107.66 155.64) (width 0.2) (layer "F.Cu") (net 31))
 (segment (start 108.26 158.94) (end 108.26 157.664999) (width 0.2) (layer "F.Cu") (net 2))
 (segment (start 108.235 156.110001) (end 108.36 155.985001) (width 0.2) (layer "F.Cu") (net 2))
 (segment (start 108.36 155.985001) (end 108.36 155.64) (width 0.2) (layer "F.Cu") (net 2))
 (segment (start 108.235 157.639999) (end 108.235 156.110001) (width 0.2) (layer "F.Cu") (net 2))
 (segment (start 108.26 157.664999) (end 108.235 157.639999) (width 0.2) (layer "F.Cu") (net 2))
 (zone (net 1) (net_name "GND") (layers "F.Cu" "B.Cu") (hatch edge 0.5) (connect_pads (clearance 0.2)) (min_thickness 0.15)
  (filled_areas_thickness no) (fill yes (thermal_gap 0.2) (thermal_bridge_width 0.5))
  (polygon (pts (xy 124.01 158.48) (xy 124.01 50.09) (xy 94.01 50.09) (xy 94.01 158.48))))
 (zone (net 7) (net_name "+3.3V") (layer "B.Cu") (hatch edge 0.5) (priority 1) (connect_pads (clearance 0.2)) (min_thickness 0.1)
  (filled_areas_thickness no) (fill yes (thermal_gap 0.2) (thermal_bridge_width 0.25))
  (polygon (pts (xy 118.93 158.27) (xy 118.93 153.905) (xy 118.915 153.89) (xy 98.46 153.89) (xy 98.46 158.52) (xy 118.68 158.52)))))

